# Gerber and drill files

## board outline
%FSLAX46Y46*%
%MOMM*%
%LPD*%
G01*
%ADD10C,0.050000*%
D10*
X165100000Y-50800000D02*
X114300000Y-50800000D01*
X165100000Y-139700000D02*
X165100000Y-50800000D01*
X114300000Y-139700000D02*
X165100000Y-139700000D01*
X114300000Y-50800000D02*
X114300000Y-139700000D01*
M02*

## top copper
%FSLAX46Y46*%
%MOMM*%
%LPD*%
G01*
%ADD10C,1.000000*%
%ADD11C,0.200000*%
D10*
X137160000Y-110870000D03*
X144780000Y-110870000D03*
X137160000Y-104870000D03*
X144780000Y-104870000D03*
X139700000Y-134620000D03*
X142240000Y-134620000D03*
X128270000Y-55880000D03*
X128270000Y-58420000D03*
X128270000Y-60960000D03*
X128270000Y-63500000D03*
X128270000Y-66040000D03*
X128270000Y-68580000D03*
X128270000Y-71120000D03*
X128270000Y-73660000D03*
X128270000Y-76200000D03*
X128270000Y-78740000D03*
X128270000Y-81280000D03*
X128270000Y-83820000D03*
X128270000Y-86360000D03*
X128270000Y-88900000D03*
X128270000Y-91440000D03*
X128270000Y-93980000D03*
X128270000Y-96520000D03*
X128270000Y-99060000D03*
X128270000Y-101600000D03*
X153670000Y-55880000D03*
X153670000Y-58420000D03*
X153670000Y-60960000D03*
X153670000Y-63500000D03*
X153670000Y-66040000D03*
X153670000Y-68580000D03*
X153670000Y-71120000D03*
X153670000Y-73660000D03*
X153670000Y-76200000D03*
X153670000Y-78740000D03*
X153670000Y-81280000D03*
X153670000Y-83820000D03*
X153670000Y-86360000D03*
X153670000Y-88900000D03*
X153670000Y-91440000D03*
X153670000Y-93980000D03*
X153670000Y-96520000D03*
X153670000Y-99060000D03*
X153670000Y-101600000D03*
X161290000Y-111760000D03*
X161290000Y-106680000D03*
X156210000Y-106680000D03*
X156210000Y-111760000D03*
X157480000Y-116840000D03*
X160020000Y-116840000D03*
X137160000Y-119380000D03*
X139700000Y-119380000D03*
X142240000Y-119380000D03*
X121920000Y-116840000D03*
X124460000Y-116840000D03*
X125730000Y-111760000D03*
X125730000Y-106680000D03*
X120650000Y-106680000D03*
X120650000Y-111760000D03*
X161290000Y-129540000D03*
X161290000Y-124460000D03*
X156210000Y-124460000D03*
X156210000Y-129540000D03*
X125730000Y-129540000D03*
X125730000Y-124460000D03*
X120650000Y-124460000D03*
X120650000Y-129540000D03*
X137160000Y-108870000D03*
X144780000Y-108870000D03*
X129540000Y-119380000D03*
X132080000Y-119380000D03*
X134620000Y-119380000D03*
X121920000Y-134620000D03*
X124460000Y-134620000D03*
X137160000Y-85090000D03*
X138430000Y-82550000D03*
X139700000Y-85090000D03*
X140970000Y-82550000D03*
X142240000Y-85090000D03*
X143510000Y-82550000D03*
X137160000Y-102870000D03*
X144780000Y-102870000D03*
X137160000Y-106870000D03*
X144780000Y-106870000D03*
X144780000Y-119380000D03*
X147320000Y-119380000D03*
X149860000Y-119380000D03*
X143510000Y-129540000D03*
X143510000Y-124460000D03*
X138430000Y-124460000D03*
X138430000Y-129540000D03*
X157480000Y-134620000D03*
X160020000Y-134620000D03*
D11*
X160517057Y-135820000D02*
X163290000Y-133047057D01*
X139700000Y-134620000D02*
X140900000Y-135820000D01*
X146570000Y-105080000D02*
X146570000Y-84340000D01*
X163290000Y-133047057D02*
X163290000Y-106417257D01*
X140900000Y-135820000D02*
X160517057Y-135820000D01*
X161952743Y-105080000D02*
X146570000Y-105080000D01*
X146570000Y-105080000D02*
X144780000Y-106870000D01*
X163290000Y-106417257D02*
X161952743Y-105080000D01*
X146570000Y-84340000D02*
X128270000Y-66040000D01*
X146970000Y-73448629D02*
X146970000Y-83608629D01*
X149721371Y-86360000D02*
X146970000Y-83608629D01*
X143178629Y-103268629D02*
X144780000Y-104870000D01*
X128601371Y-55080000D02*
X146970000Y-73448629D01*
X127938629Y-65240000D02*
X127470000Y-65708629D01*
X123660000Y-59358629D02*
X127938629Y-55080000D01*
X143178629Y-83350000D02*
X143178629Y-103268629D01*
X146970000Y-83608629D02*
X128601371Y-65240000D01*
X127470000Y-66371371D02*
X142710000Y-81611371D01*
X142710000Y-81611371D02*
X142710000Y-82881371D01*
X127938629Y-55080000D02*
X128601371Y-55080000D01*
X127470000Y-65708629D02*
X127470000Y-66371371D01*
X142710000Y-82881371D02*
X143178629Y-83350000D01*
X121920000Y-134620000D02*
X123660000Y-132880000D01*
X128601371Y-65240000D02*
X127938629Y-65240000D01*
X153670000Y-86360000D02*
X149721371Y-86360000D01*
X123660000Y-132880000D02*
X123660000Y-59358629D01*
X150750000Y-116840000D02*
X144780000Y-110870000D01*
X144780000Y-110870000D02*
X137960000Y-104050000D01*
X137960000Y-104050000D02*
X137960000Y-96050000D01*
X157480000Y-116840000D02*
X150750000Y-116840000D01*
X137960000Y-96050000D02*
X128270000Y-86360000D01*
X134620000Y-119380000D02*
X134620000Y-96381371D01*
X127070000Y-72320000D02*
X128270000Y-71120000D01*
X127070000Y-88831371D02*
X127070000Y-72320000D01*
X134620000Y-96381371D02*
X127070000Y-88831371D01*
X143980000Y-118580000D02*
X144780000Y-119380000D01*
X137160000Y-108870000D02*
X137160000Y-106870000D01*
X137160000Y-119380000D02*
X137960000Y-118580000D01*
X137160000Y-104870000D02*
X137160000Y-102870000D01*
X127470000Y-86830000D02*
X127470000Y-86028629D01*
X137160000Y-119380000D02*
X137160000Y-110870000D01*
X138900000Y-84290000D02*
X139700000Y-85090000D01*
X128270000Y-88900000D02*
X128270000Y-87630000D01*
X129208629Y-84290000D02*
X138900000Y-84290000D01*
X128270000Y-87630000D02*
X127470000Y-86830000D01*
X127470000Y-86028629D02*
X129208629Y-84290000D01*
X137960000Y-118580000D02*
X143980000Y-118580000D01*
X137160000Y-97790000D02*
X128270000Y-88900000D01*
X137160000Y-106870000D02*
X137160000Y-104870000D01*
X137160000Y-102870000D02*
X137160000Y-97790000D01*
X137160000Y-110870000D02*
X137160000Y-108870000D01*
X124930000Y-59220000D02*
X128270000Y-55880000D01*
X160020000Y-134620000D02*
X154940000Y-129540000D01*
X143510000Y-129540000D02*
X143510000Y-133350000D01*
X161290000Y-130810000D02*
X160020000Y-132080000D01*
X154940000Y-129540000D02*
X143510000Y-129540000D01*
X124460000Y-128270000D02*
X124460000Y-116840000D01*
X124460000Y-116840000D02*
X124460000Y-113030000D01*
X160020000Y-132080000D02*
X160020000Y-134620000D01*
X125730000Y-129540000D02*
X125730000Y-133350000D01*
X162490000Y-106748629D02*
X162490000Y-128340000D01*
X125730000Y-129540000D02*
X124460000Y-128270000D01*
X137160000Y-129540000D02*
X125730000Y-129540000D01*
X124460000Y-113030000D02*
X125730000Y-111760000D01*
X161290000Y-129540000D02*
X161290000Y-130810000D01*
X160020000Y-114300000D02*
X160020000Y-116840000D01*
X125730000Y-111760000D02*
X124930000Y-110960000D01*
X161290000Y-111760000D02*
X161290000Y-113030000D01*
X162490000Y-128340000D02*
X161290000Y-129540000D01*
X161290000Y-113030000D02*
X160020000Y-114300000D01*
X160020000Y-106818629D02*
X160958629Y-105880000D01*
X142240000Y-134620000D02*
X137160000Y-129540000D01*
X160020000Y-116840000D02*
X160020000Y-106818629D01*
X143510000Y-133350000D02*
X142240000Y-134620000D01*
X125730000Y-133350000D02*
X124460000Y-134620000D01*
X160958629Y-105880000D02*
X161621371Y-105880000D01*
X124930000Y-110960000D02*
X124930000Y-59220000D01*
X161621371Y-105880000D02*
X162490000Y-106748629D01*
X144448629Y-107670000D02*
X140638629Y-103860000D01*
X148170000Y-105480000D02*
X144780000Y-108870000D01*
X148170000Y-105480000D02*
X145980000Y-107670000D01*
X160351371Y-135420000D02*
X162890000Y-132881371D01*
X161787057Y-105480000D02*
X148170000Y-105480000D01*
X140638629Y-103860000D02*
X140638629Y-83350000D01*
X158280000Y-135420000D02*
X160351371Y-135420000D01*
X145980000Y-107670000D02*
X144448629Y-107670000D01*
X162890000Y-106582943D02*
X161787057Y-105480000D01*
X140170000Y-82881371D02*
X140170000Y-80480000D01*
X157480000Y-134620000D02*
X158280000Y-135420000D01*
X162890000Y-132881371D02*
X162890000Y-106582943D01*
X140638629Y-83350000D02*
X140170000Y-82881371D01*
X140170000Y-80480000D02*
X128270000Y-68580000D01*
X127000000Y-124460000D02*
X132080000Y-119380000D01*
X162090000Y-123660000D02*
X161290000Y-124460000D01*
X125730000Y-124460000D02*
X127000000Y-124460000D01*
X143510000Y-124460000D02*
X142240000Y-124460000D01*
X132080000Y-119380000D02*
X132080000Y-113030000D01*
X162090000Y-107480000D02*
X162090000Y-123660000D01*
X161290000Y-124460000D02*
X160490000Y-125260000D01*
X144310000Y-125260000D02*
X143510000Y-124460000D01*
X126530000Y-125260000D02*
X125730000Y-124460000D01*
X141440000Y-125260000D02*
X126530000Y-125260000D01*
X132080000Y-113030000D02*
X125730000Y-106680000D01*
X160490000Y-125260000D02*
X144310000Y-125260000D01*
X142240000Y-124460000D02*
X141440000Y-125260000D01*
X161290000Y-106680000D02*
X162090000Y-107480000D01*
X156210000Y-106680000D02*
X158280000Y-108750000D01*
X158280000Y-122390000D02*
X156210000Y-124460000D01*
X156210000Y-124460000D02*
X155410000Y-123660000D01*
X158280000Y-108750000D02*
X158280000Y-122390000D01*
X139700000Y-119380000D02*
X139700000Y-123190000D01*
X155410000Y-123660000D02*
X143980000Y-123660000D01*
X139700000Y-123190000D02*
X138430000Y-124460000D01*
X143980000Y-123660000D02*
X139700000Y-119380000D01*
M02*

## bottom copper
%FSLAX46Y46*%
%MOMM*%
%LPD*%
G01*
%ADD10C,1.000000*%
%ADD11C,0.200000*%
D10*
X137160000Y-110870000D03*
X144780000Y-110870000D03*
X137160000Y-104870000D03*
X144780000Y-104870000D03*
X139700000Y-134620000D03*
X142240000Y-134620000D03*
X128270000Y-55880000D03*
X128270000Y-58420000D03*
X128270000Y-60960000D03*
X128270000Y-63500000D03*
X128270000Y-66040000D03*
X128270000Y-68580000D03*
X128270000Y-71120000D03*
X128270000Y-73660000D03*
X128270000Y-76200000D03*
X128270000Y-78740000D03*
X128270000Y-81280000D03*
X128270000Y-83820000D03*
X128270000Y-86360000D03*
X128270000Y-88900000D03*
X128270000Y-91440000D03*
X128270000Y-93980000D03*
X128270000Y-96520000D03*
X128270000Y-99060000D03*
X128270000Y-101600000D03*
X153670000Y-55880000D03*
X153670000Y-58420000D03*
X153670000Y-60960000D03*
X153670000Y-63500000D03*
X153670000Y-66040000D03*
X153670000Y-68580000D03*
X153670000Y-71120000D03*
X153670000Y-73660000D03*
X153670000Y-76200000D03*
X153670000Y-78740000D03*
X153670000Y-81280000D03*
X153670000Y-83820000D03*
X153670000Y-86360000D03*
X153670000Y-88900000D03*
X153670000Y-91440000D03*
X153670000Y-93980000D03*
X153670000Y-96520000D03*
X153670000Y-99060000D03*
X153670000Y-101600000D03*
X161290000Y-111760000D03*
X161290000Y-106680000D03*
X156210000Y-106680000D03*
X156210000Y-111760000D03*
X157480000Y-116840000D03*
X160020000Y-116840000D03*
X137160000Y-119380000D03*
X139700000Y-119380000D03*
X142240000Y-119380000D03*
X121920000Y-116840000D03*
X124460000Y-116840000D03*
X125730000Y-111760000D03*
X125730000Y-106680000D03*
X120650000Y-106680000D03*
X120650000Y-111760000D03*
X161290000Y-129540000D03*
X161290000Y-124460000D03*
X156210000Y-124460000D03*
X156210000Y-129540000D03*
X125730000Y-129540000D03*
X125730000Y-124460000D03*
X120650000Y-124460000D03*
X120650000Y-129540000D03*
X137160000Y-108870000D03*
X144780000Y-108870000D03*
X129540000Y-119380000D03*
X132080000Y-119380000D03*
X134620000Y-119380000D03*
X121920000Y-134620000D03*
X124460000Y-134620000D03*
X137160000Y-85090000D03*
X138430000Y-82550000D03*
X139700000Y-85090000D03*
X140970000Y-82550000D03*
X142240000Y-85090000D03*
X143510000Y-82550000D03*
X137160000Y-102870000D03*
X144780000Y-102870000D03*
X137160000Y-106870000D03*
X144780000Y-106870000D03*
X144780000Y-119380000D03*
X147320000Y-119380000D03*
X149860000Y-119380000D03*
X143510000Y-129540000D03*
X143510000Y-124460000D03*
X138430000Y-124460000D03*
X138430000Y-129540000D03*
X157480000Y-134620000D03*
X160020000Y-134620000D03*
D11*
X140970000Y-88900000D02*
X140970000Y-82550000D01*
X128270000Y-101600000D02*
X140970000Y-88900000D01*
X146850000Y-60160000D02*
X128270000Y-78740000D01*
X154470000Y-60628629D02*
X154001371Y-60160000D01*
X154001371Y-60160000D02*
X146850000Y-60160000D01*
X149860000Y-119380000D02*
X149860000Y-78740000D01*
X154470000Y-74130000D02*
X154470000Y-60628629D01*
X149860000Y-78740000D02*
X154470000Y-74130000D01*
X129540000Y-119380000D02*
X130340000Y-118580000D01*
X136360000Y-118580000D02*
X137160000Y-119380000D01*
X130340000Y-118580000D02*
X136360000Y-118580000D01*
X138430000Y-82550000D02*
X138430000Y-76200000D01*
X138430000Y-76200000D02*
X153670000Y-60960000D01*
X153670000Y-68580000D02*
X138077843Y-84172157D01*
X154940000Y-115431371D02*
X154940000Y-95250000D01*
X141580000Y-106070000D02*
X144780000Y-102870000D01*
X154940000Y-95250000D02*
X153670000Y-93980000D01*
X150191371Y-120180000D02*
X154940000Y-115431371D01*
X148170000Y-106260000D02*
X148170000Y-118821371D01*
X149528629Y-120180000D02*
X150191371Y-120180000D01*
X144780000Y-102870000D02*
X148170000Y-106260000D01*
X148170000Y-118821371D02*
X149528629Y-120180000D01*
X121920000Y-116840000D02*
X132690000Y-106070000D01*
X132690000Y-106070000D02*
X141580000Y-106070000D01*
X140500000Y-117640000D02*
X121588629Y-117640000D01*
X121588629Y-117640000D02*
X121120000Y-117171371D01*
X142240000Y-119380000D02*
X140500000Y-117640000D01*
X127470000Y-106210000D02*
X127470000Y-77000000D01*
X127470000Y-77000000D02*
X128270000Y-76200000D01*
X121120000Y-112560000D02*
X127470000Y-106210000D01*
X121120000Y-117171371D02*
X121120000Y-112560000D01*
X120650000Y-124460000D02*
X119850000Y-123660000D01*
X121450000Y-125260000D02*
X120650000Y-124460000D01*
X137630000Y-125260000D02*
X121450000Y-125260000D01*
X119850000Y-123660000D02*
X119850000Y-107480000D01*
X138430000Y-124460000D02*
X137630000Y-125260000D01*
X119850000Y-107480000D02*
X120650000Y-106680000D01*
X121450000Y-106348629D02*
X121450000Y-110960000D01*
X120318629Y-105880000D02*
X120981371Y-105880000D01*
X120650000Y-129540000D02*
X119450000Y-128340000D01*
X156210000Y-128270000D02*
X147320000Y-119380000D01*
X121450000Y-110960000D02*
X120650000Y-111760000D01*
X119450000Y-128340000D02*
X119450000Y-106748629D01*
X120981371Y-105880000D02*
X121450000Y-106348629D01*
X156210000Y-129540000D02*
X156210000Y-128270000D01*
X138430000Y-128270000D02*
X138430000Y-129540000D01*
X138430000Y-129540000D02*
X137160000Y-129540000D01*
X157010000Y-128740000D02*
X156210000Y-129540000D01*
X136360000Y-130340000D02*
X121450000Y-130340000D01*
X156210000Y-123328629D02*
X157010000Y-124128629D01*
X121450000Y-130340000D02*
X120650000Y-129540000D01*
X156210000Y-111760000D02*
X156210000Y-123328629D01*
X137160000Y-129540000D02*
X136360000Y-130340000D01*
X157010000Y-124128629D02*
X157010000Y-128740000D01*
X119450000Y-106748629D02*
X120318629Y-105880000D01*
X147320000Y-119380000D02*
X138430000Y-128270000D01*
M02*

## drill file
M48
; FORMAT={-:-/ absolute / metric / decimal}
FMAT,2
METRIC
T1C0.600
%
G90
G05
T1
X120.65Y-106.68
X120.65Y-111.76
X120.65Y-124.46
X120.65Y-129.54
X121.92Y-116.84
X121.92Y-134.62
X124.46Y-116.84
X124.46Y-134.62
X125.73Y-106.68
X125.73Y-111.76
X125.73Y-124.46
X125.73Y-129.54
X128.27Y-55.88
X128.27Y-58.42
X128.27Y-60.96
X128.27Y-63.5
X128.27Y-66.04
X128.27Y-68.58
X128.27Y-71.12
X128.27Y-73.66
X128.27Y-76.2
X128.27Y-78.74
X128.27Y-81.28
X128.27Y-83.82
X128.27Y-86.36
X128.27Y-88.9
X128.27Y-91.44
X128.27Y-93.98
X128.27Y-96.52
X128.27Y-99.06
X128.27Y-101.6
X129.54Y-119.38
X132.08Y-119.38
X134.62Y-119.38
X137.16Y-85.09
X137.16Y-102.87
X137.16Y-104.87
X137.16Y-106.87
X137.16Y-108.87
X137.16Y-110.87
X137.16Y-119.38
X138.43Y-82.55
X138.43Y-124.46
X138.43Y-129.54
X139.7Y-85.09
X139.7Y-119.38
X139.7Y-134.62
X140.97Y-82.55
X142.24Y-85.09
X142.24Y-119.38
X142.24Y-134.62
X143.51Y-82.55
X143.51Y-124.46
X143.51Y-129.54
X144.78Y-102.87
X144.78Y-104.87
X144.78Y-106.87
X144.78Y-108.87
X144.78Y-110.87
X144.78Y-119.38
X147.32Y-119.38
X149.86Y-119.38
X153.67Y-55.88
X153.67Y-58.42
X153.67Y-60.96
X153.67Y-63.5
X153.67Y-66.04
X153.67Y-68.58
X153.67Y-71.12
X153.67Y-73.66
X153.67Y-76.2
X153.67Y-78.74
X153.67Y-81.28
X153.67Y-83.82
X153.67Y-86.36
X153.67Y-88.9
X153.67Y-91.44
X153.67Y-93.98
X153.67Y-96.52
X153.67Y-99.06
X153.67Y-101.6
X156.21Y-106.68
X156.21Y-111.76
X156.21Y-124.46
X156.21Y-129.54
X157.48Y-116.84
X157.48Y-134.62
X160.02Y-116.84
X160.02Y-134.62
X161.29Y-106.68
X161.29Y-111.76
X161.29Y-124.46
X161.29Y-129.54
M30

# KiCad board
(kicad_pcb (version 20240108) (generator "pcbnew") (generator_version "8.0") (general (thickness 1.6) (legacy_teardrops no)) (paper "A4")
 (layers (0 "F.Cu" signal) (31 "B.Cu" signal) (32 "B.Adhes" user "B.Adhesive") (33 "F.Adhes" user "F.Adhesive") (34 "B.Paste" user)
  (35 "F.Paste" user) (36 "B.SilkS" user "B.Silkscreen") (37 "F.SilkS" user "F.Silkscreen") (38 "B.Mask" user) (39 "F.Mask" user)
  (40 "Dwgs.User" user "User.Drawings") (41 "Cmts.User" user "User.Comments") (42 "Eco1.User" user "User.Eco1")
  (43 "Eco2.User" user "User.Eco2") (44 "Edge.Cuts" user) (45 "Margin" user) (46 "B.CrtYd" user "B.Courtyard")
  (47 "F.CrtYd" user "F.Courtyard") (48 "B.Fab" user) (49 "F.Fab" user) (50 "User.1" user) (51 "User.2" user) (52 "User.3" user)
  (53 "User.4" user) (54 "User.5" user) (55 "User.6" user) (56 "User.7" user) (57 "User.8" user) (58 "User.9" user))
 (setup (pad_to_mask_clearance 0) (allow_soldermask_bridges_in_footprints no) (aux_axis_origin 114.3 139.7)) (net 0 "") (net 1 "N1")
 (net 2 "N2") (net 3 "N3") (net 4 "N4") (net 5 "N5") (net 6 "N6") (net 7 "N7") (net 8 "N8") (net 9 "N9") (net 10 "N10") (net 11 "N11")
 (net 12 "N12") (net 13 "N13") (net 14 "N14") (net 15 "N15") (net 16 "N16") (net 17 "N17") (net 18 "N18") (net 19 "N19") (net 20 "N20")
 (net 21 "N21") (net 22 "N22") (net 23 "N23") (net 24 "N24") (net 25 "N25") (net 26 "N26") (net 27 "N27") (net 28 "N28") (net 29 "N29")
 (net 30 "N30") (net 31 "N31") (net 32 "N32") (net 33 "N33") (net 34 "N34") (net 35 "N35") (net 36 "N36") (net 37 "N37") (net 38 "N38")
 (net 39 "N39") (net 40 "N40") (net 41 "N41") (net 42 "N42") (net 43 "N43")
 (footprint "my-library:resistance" (layer "F.Cu") (at 139.7 110.87)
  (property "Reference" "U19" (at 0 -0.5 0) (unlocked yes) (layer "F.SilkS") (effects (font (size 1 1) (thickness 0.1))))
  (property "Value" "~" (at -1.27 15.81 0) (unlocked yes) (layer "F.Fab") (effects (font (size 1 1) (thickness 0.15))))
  (pad "1" thru_hole circle (at -2.54 0) (size 1 1) (drill 0.6) (layers "*.Cu" "*.Mask") (remove_unused_layers no) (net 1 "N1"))
  (pad "2" thru_hole circle (at 5.08 0) (size 1 1) (drill 0.6) (layers "*.Cu" "*.Mask") (remove_unused_layers no) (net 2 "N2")))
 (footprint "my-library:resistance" (layer "F.Cu") (at 139.7 104.87)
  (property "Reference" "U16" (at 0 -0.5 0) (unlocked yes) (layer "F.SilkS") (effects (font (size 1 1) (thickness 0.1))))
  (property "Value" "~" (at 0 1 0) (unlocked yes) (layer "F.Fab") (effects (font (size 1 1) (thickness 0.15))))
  (pad "1" thru_hole circle (at -2.54 0) (size 1 1) (drill 0.6) (layers "*.Cu" "*.Mask") (remove_unused_layers no) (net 1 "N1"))
  (pad "2" thru_hole circle (at 5.08 0) (size 1 1) (drill 0.6) (layers "*.Cu" "*.Mask") (remove_unused_layers no) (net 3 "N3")))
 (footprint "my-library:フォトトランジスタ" (layer "F.Cu") (at 139.7 134.62)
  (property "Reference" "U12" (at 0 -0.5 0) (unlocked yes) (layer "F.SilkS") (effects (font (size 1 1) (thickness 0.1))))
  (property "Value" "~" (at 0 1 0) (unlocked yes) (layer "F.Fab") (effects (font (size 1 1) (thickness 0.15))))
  (pad "1" thru_hole circle (at 0 0) (size 1 1) (drill 0.6) (layers "*.Cu" "*.Mask") (remove_unused_layers no) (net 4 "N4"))
  (pad "2" thru_hole circle (at 2.54 0) (size 1 1) (drill 0.6) (layers "*.Cu" "*.Mask") (remove_unused_layers no) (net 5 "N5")))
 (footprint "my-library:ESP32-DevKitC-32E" (layer "F.Cu") (at 140.97 76.2)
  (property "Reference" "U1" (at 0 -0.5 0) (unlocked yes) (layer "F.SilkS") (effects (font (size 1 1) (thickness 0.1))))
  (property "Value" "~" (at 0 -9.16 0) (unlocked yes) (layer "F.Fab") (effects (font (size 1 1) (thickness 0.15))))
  (pad "1" thru_hole circle (at -12.7 -20.32) (size 1 1) (drill 0.6) (layers "*.Cu" "*.Mask") (remove_unused_layers no) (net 5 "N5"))
  (pad "2" thru_hole circle (at -12.7 -17.78) (size 1 1) (drill 0.6) (layers "*.Cu" "*.Mask") (remove_unused_layers no) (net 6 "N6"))
  (pad "3" thru_hole circle (at -12.7 -15.24) (size 1 1) (drill 0.6) (layers "*.Cu" "*.Mask") (remove_unused_layers no) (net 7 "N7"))
  (pad "4" thru_hole circle (at -12.7 -12.7) (size 1 1) (drill 0.6) (layers "*.Cu" "*.Mask") (remove_unused_layers no) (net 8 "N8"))
  (pad "5" thru_hole circle (at -12.7 -10.16) (size 1 1) (drill 0.6) (layers "*.Cu" "*.Mask") (remove_unused_layers no) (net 4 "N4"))
  (pad "6" thru_hole circle (at -12.7 -7.62) (size 1 1) (drill 0.6) (layers "*.Cu" "*.Mask") (remove_unused_layers no) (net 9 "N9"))
  (pad "7" thru_hole circle (at -12.7 -5.08) (size 1 1) (drill 0.6) (layers "*.Cu" "*.Mask") (remove_unused_layers no) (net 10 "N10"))
  (pad "8" thru_hole circle (at -12.7 -2.54) (size 1 1) (drill 0.6) (layers "*.Cu" "*.Mask") (remove_unused_layers no) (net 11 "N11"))
  (pad "9" thru_hole circle (at -12.7 0) (size 1 1) (drill 0.6) (layers "*.Cu" "*.Mask") (remove_unused_layers no) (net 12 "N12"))
  (pad "10" thru_hole circle (at -12.7 2.54) (size 1 1) (drill 0.6) (layers "*.Cu" "*.Mask") (remove_unused_layers no) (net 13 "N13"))
  (pad "11" thru_hole circle (at -12.7 5.08) (size 1 1) (drill 0.6) (layers "*.Cu" "*.Mask") (remove_unused_layers no) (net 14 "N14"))
  (pad "12" thru_hole circle (at -12.7 7.62) (size 1 1) (drill 0.6) (layers "*.Cu" "*.Mask") (remove_unused_layers no) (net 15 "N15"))
  (pad "13" thru_hole circle (at -12.7 10.16) (size 1 1) (drill 0.6) (layers "*.Cu" "*.Mask") (remove_unused_layers no) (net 2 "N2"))
  (pad "14" thru_hole circle (at -12.7 12.7) (size 1 1) (drill 0.6) (layers "*.Cu" "*.Mask") (remove_unused_layers no) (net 1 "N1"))
  (pad "15" thru_hole circle (at -12.7 15.24) (size 1 1) (drill 0.6) (layers "*.Cu" "*.Mask") (remove_unused_layers no) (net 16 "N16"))
  (pad "16" thru_hole circle (at -12.7 17.78) (size 1 1) (drill 0.6) (layers "*.Cu" "*.Mask") (remove_unused_layers no) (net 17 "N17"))
  (pad "17" thru_hole circle (at -12.7 20.32) (size 1 1) (drill 0.6) (layers "*.Cu" "*.Mask") (remove_unused_layers no) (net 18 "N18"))
  (pad "18" thru_hole circle (at -12.7 22.86) (size 1 1) (drill 0.6) (layers "*.Cu" "*.Mask") (remove_unused_layers no) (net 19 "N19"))
  (pad "19" thru_hole circle (at -12.7 25.4) (size 1 1) (drill 0.6) (layers "*.Cu" "*.Mask") (remove_unused_layers no) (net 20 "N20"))
  (pad "20" thru_hole circle (at 12.7 -20.32) (size 1 1) (drill 0.6) (layers "*.Cu" "*.Mask") (remove_unused_layers no) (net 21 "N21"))
  (pad "21" thru_hole circle (at 12.7 -17.78) (size 1 1) (drill 0.6) (layers "*.Cu" "*.Mask") (remove_unused_layers no) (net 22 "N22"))
  (pad "22" thru_hole circle (at 12.7 -15.24) (size 1 1) (drill 0.6) (layers "*.Cu" "*.Mask") (remove_unused_layers no) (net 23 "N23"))
  (pad "23" thru_hole circle (at 12.7 -12.7) (size 1 1) (drill 0.6) (layers "*.Cu" "*.Mask") (remove_unused_layers no) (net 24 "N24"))
  (pad "24" thru_hole circle (at 12.7 -10.16) (size 1 1) (drill 0.6) (layers "*.Cu" "*.Mask") (remove_unused_layers no) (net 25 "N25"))
  (pad "25" thru_hole circle (at 12.7 -7.62) (size 1 1) (drill 0.6) (layers "*.Cu" "*.Mask") (remove_unused_layers no) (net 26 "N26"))
  (pad "26" thru_hole circle (at 12.7 -5.08) (size 1 1) (drill 0.6) (layers "*.Cu" "*.Mask") (remove_unused_layers no) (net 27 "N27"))
  (pad "27" thru_hole circle (at 12.7 -2.54) (size 1 1) (drill 0.6) (layers "*.Cu" "*.Mask") (remove_unused_layers no) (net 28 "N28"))
  (pad "28" thru_hole circle (at 12.7 0) (size 1 1) (drill 0.6) (layers "*.Cu" "*.Mask") (remove_unused_layers no) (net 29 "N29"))
  (pad "29" thru_hole circle (at 12.7 2.54) (size 1 1) (drill 0.6) (layers "*.Cu" "*.Mask") (remove_unused_layers no) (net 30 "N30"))
  (pad "30" thru_hole circle (at 12.7 5.08) (size 1 1) (drill 0.6) (layers "*.Cu" "*.Mask") (remove_unused_layers no) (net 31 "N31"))
  (pad "31" thru_hole circle (at 12.7 7.62) (size 1 1) (drill 0.6) (layers "*.Cu" "*.Mask") (remove_unused_layers no) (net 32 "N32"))
  (pad "32" thru_hole circle (at 12.7 10.16) (size 1 1) (drill 0.6) (layers "*.Cu" "*.Mask") (remove_unused_layers no) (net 3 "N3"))
  (pad "33" thru_hole circle (at 12.7 12.7) (size 1 1) (drill 0.6) (layers "*.Cu" "*.Mask") (remove_unused_layers no) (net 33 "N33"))
  (pad "34" thru_hole circle (at 12.7 15.24) (size 1 1) (drill 0.6) (layers "*.Cu" "*.Mask") (remove_unused_layers no) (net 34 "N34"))
  (pad "35" thru_hole circle (at 12.7 17.78) (size 1 1) (drill 0.6) (layers "*.Cu" "*.Mask") (remove_unused_layers no) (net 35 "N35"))
  (pad "36" thru_hole circle (at 12.7 20.32) (size 1 1) (drill 0.6) (layers "*.Cu" "*.Mask") (remove_unused_layers no) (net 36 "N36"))
  (pad "37" thru_hole circle (at 12.7 22.86) (size 1 1) (drill 0.6) (layers "*.Cu" "*.Mask") (remove_unused_layers no) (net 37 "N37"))
  (pad "38" thru_hole circle (at 12.7 25.4) (size 1 1) (drill 0.6) (layers "*.Cu" "*.Mask") (remove_unused_layers no) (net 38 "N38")))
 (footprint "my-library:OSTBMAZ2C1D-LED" (layer "F.Cu") (at 158.75 109.22)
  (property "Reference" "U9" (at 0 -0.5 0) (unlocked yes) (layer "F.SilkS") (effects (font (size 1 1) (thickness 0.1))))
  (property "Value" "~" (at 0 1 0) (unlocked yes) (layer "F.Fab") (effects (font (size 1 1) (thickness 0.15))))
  (pad "1" thru_hole circle (at 2.54 2.54) (size 1 1) (drill 0.6) (layers "*.Cu" "*.Mask") (remove_unused_layers no) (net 5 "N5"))
  (pad "2" thru_hole circle (at 2.54 -2.54) (size 1 1) (drill 0.6) (layers "*.Cu" "*.Mask") (remove_unused_layers no) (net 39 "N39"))
  (pad "3" thru_hole circle (at -2.54 -2.54) (size 1 1) (drill 0.6) (layers "*.Cu" "*.Mask") (remove_unused_layers no) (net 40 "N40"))
  (pad "4" thru_hole circle (at -2.54 2.54) (size 1 1) (drill 0.6) (layers "*.Cu" "*.Mask") (remove_unused_layers no) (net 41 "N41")))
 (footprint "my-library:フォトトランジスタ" (layer "F.Cu") (at 157.48 116.84)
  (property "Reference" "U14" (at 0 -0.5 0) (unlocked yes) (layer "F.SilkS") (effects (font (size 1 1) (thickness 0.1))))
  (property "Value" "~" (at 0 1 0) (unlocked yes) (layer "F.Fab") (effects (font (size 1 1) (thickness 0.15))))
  (pad "1" thru_hole circle (at 0 0) (size 1 1) (drill 0.6) (layers "*.Cu" "*.Mask") (remove_unused_layers no) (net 2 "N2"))
  (pad "2" thru_hole circle (at 2.54 0) (size 1 1) (drill 0.6) (layers "*.Cu" "*.Mask") (remove_unused_layers no) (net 5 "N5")))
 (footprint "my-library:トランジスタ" (layer "F.Cu") (at 139.7 116.84)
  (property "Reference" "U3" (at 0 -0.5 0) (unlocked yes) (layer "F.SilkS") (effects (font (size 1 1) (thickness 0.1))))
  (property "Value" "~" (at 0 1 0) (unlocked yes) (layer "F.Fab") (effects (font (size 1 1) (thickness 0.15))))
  (pad "1" thru_hole circle (at -2.54 2.54) (size 1 1) (drill 0.6) (layers "*.Cu" "*.Mask") (remove_unused_layers no) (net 1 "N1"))
  (pad "2" thru_hole circle (at 0 2.54) (size 1 1) (drill 0.6) (layers "*.Cu" "*.Mask") (remove_unused_layers no) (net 40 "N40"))
  (pad "3" thru_hole circle (at 2.54 2.54) (size 1 1) (drill 0.6) (layers "*.Cu" "*.Mask") (remove_unused_layers no) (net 12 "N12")))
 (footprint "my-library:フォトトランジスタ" (layer "F.Cu") (at 121.92 116.84)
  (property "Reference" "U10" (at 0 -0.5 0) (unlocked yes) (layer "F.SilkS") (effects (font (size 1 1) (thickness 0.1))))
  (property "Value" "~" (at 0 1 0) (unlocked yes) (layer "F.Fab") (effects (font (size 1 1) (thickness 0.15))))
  (pad "1" thru_hole circle (at 0 0) (size 1 1) (drill 0.6) (layers "*.Cu" "*.Mask") (remove_unused_layers no) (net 35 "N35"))
  (pad "2" thru_hole circle (at 2.54 0) (size 1 1) (drill 0.6) (layers "*.Cu" "*.Mask") (remove_unused_layers no) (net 5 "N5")))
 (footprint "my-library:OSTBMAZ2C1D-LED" (layer "F.Cu") (at 123.19 109.22)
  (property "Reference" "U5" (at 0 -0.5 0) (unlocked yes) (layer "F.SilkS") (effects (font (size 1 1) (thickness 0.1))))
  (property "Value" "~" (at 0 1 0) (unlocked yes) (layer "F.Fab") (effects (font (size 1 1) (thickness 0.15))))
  (pad "1" thru_hole circle (at 2.54 2.54) (size 1 1) (drill 0.6) (layers "*.Cu" "*.Mask") (remove_unused_layers no) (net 5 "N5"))
  (pad "2" thru_hole circle (at 2.54 -2.54) (size 1 1) (drill 0.6) (layers "*.Cu" "*.Mask") (remove_unused_layers no) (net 39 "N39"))
  (pad "3" thru_hole circle (at -2.54 -2.54) (size 1 1) (drill 0.6) (layers "*.Cu" "*.Mask") (remove_unused_layers no) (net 40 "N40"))
  (pad "4" thru_hole circle (at -2.54 2.54) (size 1 1) (drill 0.6) (layers "*.Cu" "*.Mask") (remove_unused_layers no) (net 41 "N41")))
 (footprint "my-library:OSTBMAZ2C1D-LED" (layer "F.Cu") (at 158.75 127)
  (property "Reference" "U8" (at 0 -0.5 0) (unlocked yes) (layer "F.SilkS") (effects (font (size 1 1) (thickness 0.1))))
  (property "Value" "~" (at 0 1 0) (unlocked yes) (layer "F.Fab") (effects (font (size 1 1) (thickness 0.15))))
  (pad "1" thru_hole circle (at 2.54 2.54) (size 1 1) (drill 0.6) (layers "*.Cu" "*.Mask") (remove_unused_layers no) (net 5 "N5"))
  (pad "2" thru_hole circle (at 2.54 -2.54) (size 1 1) (drill 0.6) (layers "*.Cu" "*.Mask") (remove_unused_layers no) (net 39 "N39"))
  (pad "3" thru_hole circle (at -2.54 -2.54) (size 1 1) (drill 0.6) (layers "*.Cu" "*.Mask") (remove_unused_layers no) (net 40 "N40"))
  (pad "4" thru_hole circle (at -2.54 2.54) (size 1 1) (drill 0.6) (layers "*.Cu" "*.Mask") (remove_unused_layers no) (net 41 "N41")))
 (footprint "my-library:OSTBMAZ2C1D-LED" (layer "F.Cu") (at 123.19 127)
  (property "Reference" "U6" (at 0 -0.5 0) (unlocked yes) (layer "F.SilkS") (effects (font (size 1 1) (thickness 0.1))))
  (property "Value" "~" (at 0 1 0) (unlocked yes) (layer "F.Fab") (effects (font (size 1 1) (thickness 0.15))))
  (pad "1" thru_hole circle (at 2.54 2.54) (size 1 1) (drill 0.6) (layers "*.Cu" "*.Mask") (remove_unused_layers no) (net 5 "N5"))
  (pad "2" thru_hole circle (at 2.54 -2.54) (size 1 1) (drill 0.6) (layers "*.Cu" "*.Mask") (remove_unused_layers no) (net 39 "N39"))
  (pad "3" thru_hole circle (at -2.54 -2.54) (size 1 1) (drill 0.6) (layers "*.Cu" "*.Mask") (remove_unused_layers no) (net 40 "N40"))
  (pad "4" thru_hole circle (at -2.54 2.54) (size 1 1) (drill 0.6) (layers "*.Cu" "*.Mask") (remove_unused_layers no) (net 41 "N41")))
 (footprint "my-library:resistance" (layer "F.Cu") (at 139.7 108.87)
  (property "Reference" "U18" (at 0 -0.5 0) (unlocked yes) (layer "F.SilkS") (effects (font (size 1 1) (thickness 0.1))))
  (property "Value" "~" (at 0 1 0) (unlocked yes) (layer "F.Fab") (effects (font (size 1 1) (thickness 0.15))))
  (pad "1" thru_hole circle (at -2.54 0) (size 1 1) (drill 0.6) (layers "*.Cu" "*.Mask") (remove_unused_layers no) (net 1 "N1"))
  (pad "2" thru_hole circle (at 5.08 0) (size 1 1) (drill 0.6) (layers "*.Cu" "*.Mask") (remove_unused_layers no) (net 9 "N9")))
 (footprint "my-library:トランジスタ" (layer "F.Cu") (at 132.08 116.84)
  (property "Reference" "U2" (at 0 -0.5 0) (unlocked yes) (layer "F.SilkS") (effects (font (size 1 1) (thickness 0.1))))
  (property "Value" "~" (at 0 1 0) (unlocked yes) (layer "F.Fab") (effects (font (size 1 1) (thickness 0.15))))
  (pad "1" thru_hole circle (at -2.54 2.54) (size 1 1) (drill 0.6) (layers "*.Cu" "*.Mask") (remove_unused_layers no) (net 1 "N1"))
  (pad "2" thru_hole circle (at 0 2.54) (size 1 1) (drill 0.6) (layers "*.Cu" "*.Mask") (remove_unused_layers no) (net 39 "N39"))
  (pad "3" thru_hole circle (at 2.54 2.54) (size 1 1) (drill 0.6) (layers "*.Cu" "*.Mask") (remove_unused_layers no) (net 10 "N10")))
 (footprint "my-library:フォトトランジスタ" (layer "F.Cu") (at 121.92 134.62)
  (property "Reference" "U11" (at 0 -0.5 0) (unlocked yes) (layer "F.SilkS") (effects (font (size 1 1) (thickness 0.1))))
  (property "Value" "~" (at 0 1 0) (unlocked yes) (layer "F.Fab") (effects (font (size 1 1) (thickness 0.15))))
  (pad "1" thru_hole circle (at 0 0) (size 1 1) (drill 0.6) (layers "*.Cu" "*.Mask") (remove_unused_layers no) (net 3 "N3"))
  (pad "2" thru_hole circle (at 2.54 0) (size 1 1) (drill 0.6) (layers "*.Cu" "*.Mask") (remove_unused_layers no) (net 5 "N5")))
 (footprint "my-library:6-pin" (layer "F.Cu") (at 139.7 82.55)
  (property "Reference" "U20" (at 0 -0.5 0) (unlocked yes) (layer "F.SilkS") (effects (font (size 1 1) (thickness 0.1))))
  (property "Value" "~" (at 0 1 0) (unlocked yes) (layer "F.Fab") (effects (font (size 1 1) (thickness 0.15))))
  (pad "1" thru_hole circle (at -2.54 2.54) (size 1 1) (drill 0.6) (layers "*.Cu" "*.Mask") (remove_unused_layers no) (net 26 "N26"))
  (pad "2" thru_hole circle (at -1.27 0) (size 1 1) (drill 0.6) (layers "*.Cu" "*.Mask") (remove_unused_layers no) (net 23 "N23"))
  (pad "3" thru_hole circle (at 0 2.54) (size 1 1) (drill 0.6) (layers "*.Cu" "*.Mask") (remove_unused_layers no) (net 1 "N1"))
  (pad "4" thru_hole circle (at 1.27 0) (size 1 1) (drill 0.6) (layers "*.Cu" "*.Mask") (remove_unused_layers no) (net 20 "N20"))
  (pad "5" thru_hole circle (at 2.54 2.54) (size 1 1) (drill 0.6) (layers "*.Cu" "*.Mask") (remove_unused_layers no) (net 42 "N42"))
  (pad "6" thru_hole circle (at 3.81 0) (size 1 1) (drill 0.6) (layers "*.Cu" "*.Mask") (remove_unused_layers no) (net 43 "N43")))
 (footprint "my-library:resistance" (layer "F.Cu") (at 139.7 102.87)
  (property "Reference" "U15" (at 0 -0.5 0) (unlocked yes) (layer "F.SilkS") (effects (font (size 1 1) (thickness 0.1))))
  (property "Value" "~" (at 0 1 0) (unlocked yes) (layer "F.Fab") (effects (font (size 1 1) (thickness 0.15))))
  (pad "1" thru_hole circle (at -2.54 0) (size 1 1) (drill 0.6) (layers "*.Cu" "*.Mask") (remove_unused_layers no) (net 1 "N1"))
  (pad "2" thru_hole circle (at 5.08 0) (size 1 1) (drill 0.6) (layers "*.Cu" "*.Mask") (remove_unused_layers no) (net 35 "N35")))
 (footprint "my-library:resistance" (layer "F.Cu") (at 139.7 106.87)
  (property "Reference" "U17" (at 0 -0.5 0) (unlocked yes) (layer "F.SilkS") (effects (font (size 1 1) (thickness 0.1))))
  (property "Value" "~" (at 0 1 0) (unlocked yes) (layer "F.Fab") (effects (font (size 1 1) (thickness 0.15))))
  (pad "1" thru_hole circle (at -2.54 0) (size 1 1) (drill 0.6) (layers "*.Cu" "*.Mask") (remove_unused_layers no) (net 1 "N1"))
  (pad "2" thru_hole circle (at 5.08 0) (size 1 1) (drill 0.6) (layers "*.Cu" "*.Mask") (remove_unused_layers no) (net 4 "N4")))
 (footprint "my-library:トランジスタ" (layer "F.Cu") (at 147.32 116.84)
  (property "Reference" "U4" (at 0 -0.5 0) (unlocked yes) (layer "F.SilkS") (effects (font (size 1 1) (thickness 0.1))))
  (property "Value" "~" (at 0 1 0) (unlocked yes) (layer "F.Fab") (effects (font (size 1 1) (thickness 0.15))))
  (pad "1" thru_hole circle (at -2.54 2.54) (size 1 1) (drill 0.6) (layers "*.Cu" "*.Mask") (remove_unused_layers no) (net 1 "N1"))
  (pad "2" thru_hole circle (at 0 2.54) (size 1 1) (drill 0.6) (layers "*.Cu" "*.Mask") (remove_unused_layers no) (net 41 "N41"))
  (pad "3" thru_hole circle (at 2.54 2.54) (size 1 1) (drill 0.6) (layers "*.Cu" "*.Mask") (remove_unused_layers no) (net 13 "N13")))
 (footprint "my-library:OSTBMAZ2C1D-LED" (layer "F.Cu") (at 140.97 127)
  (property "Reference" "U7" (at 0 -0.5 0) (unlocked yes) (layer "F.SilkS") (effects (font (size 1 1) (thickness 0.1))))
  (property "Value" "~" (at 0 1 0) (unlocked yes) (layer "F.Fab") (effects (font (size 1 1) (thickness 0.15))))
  (pad "1" thru_hole circle (at 2.54 2.54) (size 1 1) (drill 0.6) (layers "*.Cu" "*.Mask") (remove_unused_layers no) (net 5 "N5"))
  (pad "2" thru_hole circle (at 2.54 -2.54) (size 1 1) (drill 0.6) (layers "*.Cu" "*.Mask") (remove_unused_layers no) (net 39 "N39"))
  (pad "3" thru_hole circle (at -2.54 -2.54) (size 1 1) (drill 0.6) (layers "*.Cu" "*.Mask") (remove_unused_layers no) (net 40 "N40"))
  (pad "4" thru_hole circle (at -2.54 2.54) (size 1 1) (drill 0.6) (layers "*.Cu" "*.Mask") (remove_unused_layers no) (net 41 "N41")))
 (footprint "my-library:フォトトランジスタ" (layer "F.Cu") (at 157.48 134.62)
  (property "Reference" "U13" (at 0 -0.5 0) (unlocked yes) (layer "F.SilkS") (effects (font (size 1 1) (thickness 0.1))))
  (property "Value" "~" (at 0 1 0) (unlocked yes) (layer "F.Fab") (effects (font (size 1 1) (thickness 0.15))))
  (pad "1" thru_hole circle (at 0 0) (size 1 1) (drill 0.6) (layers "*.Cu" "*.Mask") (remove_unused_layers no) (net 9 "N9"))
  (pad "2" thru_hole circle (at 2.54 0) (size 1 1) (drill 0.6) (layers "*.Cu" "*.Mask") (remove_unused_layers no) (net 5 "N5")))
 (gr_line (start 165.1 50.8) (end 114.3 50.8) (stroke (width 0.05) (type default)) (layer "Edge.Cuts"))
 (gr_line (start 165.1 139.7) (end 165.1 50.8) (stroke (width 0.05) (type default)) (layer "Edge.Cuts"))
 (gr_line (start 114.3 139.7) (end 165.1 139.7) (stroke (width 0.05) (type default)) (layer "Edge.Cuts"))
 (gr_line (start 114.3 50.8) (end 114.3 139.7) (stroke (width 0.05) (type default)) (layer "Edge.Cuts"))
 (segment (start 140.97 88.9) (end 140.97 82.55) (width 0.2) (layer "B.Cu") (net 20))
 (segment (start 128.27 101.6) (end 140.97 88.9) (width 0.2) (layer "B.Cu") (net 20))
 (segment (start 160.517057 135.82) (end 163.29 133.047057) (width 0.2) (layer "F.Cu") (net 4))
 (segment (start 139.7 134.62) (end 140.9 135.82) (width 0.2) (layer "F.Cu") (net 4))
 (segment (start 146.57 105.08) (end 146.57 84.34) (width 0.2) (layer "F.Cu") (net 4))
 (segment (start 163.29 133.047057) (end 163.29 106.417257) (width 0.2) (layer "F.Cu") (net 4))
 (segment (start 140.9 135.82) (end 160.517057 135.82) (width 0.2) (layer "F.Cu") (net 4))
 (segment (start 161.952743 105.08) (end 146.57 105.08) (width 0.2) (layer "F.Cu") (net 4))
 (segment (start 146.57 105.08) (end 144.78 106.87) (width 0.2) (layer "F.Cu") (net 4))
 (segment (start 163.29 106.417257) (end 161.952743 105.08) (width 0.2) (layer "F.Cu") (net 4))
 (segment (start 146.57 84.34) (end 128.27 66.04) (width 0.2) (layer "F.Cu") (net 4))
 (segment (start 146.97 73.448629) (end 146.97 83.608629) (width 0.2) (layer "F.Cu") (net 3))
 (segment (start 149.721371 86.36) (end 146.97 83.608629) (width 0.2) (layer "F.Cu") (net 3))
 (segment (start 143.178629 103.268629) (end 144.78 104.87) (width 0.2) (layer "F.Cu") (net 3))
 (segment (start 128.601371 55.08) (end 146.97 73.448629) (width 0.2) (layer "F.Cu") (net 3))
 (segment (start 127.938629 65.24) (end 127.47 65.708629) (width 0.2) (layer "F.Cu") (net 3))
 (segment (start 123.66 59.358629) (end 127.938629 55.08) (width 0.2) (layer "F.Cu") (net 3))
 (segment (start 143.178629 83.35) (end 143.178629 103.268629) (width 0.2) (layer "F.Cu") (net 3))
 (segment (start 146.97 83.608629) (end 128.601371 65.24) (width 0.2) (layer "F.Cu") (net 3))
 (segment (start 127.47 66.371371) (end 142.71 81.611371) (width 0.2) (layer "F.Cu") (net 3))
 (segment (start 142.71 81.611371) (end 142.71 82.881371) (width 0.2) (layer "F.Cu") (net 3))
 (segment (start 127.938629 55.08) (end 128.601371 55.08) (width 0.2) (layer "F.Cu") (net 3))
 (segment (start 127.47 65.708629) (end 127.47 66.371371) (width 0.2) (layer "F.Cu") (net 3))
 (segment (start 142.71 82.881371) (end 143.178629 83.35) (width 0.2) (layer "F.Cu") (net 3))
 (segment (start 121.92 134.62) (end 123.66 132.88) (width 0.2) (layer "F.Cu") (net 3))
 (segment (start 128.601371 65.24) (end 127.938629 65.24) (width 0.2) (layer "F.Cu") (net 3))
 (segment (start 153.67 86.36) (end 149.721371 86.36) (width 0.2) (layer "F.Cu") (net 3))
 (segment (start 123.66 132.88) (end 123.66 59.358629) (width 0.2) (layer "F.Cu") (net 3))
 (segment (start 150.75 116.84) (end 144.78 110.87) (width 0.2) (layer "F.Cu") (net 2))
 (segment (start 144.78 110.87) (end 137.96 104.05) (width 0.2) (layer "F.Cu") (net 2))
 (segment (start 137.96 104.05) (end 137.96 96.05) (width 0.2) (layer "F.Cu") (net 2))
 (segment (start 157.48 116.84) (end 150.75 116.84) (width 0.2) (layer "F.Cu") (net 2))
 (segment (start 137.96 96.05) (end 128.27 86.36) (width 0.2) (layer "F.Cu") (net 2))
 (segment (start 146.85 60.16) (end 128.27 78.74) (width 0.2) (layer "B.Cu") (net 13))
 (segment (start 154.47 60.628629) (end 154.001371 60.16) (width 0.2) (layer "B.Cu") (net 13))
 (segment (start 154.001371 60.16) (end 146.85 60.16) (width 0.2) (layer "B.Cu") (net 13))
 (segment (start 149.86 119.38) (end 149.86 78.74) (width 0.2) (layer "B.Cu") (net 13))
 (segment (start 154.47 74.13) (end 154.47 60.628629) (width 0.2) (layer "B.Cu") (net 13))
 (segment (start 149.86 78.74) (end 154.47 74.13) (width 0.2) (layer "B.Cu") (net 13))
 (segment (start 134.62 119.38) (end 134.62 96.381371) (width 0.2) (layer "F.Cu") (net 10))
 (segment (start 127.07 72.32) (end 128.27 71.12) (width 0.2) (layer "F.Cu") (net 10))
 (segment (start 127.07 88.831371) (end 127.07 72.32) (width 0.2) (layer "F.Cu") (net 10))
 (segment (start 134.62 96.381371) (end 127.07 88.831371) (width 0.2) (layer "F.Cu") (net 10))
 (segment (start 143.98 118.58) (end 144.78 119.38) (width 0.2) (layer "F.Cu") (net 1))
 (segment (start 137.16 108.87) (end 137.16 106.87) (width 0.2) (layer "F.Cu") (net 1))
 (segment (start 137.16 119.38) (end 137.96 118.58) (width 0.2) (layer "F.Cu") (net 1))
 (segment (start 137.16 104.87) (end 137.16 102.87) (width 0.2) (layer "F.Cu") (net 1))
 (segment (start 127.47 86.83) (end 127.47 86.028629) (width 0.2) (layer "F.Cu") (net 1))
 (segment (start 137.16 119.38) (end 137.16 110.87) (width 0.2) (layer "F.Cu") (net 1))
 (segment (start 138.9 84.29) (end 139.7 85.09) (width 0.2) (layer "F.Cu") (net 1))
 (segment (start 128.27 88.9) (end 128.27 87.63) (width 0.2) (layer "F.Cu") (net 1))
 (segment (start 129.208629 84.29) (end 138.9 84.29) (width 0.2) (layer "F.Cu") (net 1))
 (segment (start 128.27 87.63) (end 127.47 86.83) (width 0.2) (layer "F.Cu") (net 1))
 (segment (start 127.47 86.028629) (end 129.208629 84.29) (width 0.2) (layer "F.Cu") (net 1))
 (segment (start 137.96 118.58) (end 143.98 118.58) (width 0.2) (layer "F.Cu") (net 1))
 (segment (start 137.16 97.79) (end 128.27 88.9) (width 0.2) (layer "F.Cu") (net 1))
 (segment (start 137.16 106.87) (end 137.16 104.87) (width 0.2) (layer "F.Cu") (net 1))
 (segment (start 137.16 102.87) (end 137.16 97.79) (width 0.2) (layer "F.Cu") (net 1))
 (segment (start 137.16 110.87) (end 137.16 108.87) (width 0.2) (layer "F.Cu") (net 1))
 (segment (start 129.54 119.38) (end 130.34 118.58) (width 0.2) (layer "B.Cu") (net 1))
 (segment (start 136.36 118.58) (end 137.16 119.38) (width 0.2) (layer "B.Cu") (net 1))
 (segment (start 130.34 118.58) (end 136.36 118.58) (width 0.2) (layer "B.Cu") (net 1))
 (segment (start 124.93 59.22) (end 128.27 55.88) (width 0.2) (layer "F.Cu") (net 5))
 (segment (start 160.02 134.62) (end 154.94 129.54) (width 0.2) (layer "F.Cu") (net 5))
 (segment (start 143.51 129.54) (end 143.51 133.35) (width 0.2) (layer "F.Cu") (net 5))
 (segment (start 161.29 130.81) (end 160.02 132.08) (width 0.2) (layer "F.Cu") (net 5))
 (segment (start 154.94 129.54) (end 143.51 129.54) (width 0.2) (layer "F.Cu") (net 5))
 (segment (start 124.46 128.27) (end 124.46 116.84) (width 0.2) (layer "F.Cu") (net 5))
 (segment (start 124.46 116.84) (end 124.46 113.03) (width 0.2) (layer "F.Cu") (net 5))
 (segment (start 160.02 132.08) (end 160.02 134.62) (width 0.2) (layer "F.Cu") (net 5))
 (segment (start 125.73 129.54) (end 125.73 133.35) (width 0.2) (layer "F.Cu") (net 5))
 (segment (start 162.49 106.748629) (end 162.49 128.34) (width 0.2) (layer "F.Cu") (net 5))
 (segment (start 125.73 129.54) (end 124.46 128.27) (width 0.2) (layer "F.Cu") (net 5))
 (segment (start 137.16 129.54) (end 125.73 129.54) (width 0.2) (layer "F.Cu") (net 5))
 (segment (start 124.46 113.03) (end 125.73 111.76) (width 0.2) (layer "F.Cu") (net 5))
 (segment (start 161.29 129.54) (end 161.29 130.81) (width 0.2) (layer "F.Cu") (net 5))
 (segment (start 160.02 114.3) (end 160.02 116.84) (width 0.2) (layer "F.Cu") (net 5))
 (segment (start 125.73 111.76) (end 124.93 110.96) (width 0.2) (layer "F.Cu") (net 5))
 (segment (start 161.29 111.76) (end 161.29 113.03) (width 0.2) (layer "F.Cu") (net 5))
 (segment (start 162.49 128.34) (end 161.29 129.54) (width 0.2) (layer "F.Cu") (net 5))
 (segment (start 161.29 113.03) (end 160.02 114.3) (width 0.2) (layer "F.Cu") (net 5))
 (segment (start 160.02 106.818629) (end 160.958629 105.88) (width 0.2) (layer "F.Cu") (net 5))
 (segment (start 142.24 134.62) (end 137.16 129.54) (width 0.2) (layer "F.Cu") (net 5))
 (segment (start 160.02 116.84) (end 160.02 106.818629) (width 0.2) (layer "F.Cu") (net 5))
 (segment (start 143.51 133.35) (end 142.24 134.62) (width 0.2) (layer "F.Cu") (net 5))
 (segment (start 125.73 133.35) (end 124.46 134.62) (width 0.2) (layer "F.Cu") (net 5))
 (segment (start 160.958629 105.88) (end 161.621371 105.88) (width 0.2) (layer "F.Cu") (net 5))
 (segment (start 124.93 110.96) (end 124.93 59.22) (width 0.2) (layer "F.Cu") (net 5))
 (segment (start 161.621371 105.88) (end 162.49 106.748629) (width 0.2) (layer "F.Cu") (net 5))
 (segment (start 138.43 82.55) (end 138.43 76.2) (width 0.2) (layer "B.Cu") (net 23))
 (segment (start 138.43 76.2) (end 153.67 60.96) (width 0.2) (layer "B.Cu") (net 23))
 (segment (start 153.67 68.58) (end 138.077843 84.172157) (width 0.2) (layer "B.Cu") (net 26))
 (segment (start 154.94 115.431371) (end 154.94 95.25) (width 0.2) (layer "B.Cu") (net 35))
 (segment (start 141.58 106.07) (end 144.78 102.87) (width 0.2) (layer "B.Cu") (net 35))
 (segment (start 154.94 95.25) (end 153.67 93.98) (width 0.2) (layer "B.Cu") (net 35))
 (segment (start 150.191371 120.18) (end 154.94 115.431371) (width 0.2) (layer "B.Cu") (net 35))
 (segment (start 148.17 106.26) (end 148.17 118.821371) (width 0.2) (layer "B.Cu") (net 35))
 (segment (start 149.528629 120.18) (end 150.191371 120.18) (width 0.2) (layer "B.Cu") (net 35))
 (segment (start 144.78 102.87) (end 148.17 106.26) (width 0.2) (layer "B.Cu") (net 35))
 (segment (start 148.17 118.821371) (end 149.528629 120.18) (width 0.2) (layer "B.Cu") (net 35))
 (segment (start 121.92 116.84) (end 132.69 106.07) (width 0.2) (layer "B.Cu") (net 35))
 (segment (start 132.69 106.07) (end 141.58 106.07) (width 0.2) (layer "B.Cu") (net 35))
 (segment (start 140.5 117.64) (end 121.588629 117.64) (width 0.2) (layer "B.Cu") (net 12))
 (segment (start 121.588629 117.64) (end 121.12 117.171371) (width 0.2) (layer "B.Cu") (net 12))
 (segment (start 142.24 119.38) (end 140.5 117.64) (width 0.2) (layer "B.Cu") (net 12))
 (segment (start 127.47 106.21) (end 127.47 77) (width 0.2) (layer "B.Cu") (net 12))
 (segment (start 127.47 77) (end 128.27 76.2) (width 0.2) (layer "B.Cu") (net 12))
 (segment (start 121.12 112.56) (end 127.47 106.21) (width 0.2) (layer "B.Cu") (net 12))
 (segment (start 121.12 117.171371) (end 121.12 112.56) (width 0.2) (layer "B.Cu") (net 12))
 (segment (start 144.448629 107.67) (end 140.638629 103.86) (width 0.2) (layer "F.Cu") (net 9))
 (segment (start 148.17 105.48) (end 144.78 108.87) (width 0.2) (layer "F.Cu") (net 9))
 (segment (start 148.17 105.48) (end 145.98 107.67) (width 0.2) (layer "F.Cu") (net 9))
 (segment (start 160.351371 135.42) (end 162.89 132.881371) (width 0.2) (layer "F.Cu") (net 9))
 (segment (start 161.787057 105.48) (end 148.17 105.48) (width 0.2) (layer "F.Cu") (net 9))
 (segment (start 140.638629 103.86) (end 140.638629 83.35) (width 0.2) (layer "F.Cu") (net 9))
 (segment (start 158.28 135.42) (end 160.351371 135.42) (width 0.2) (layer "F.Cu") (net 9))
 (segment (start 145.98 107.67) (end 144.448629 107.67) (width 0.2) (layer "F.Cu") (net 9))
 (segment (start 162.89 106.582943) (end 161.787057 105.48) (width 0.2) (layer "F.Cu") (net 9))
 (segment (start 140.17 82.881371) (end 140.17 80.48) (width 0.2) (layer "F.Cu") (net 9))
 (segment (start 157.48 134.62) (end 158.28 135.42) (width 0.2) (layer "F.Cu") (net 9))
 (segment (start 162.89 132.881371) (end 162.89 106.582943) (width 0.2) (layer "F.Cu") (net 9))
 (segment (start 140.638629 83.35) (end 140.17 82.881371) (width 0.2) (layer "F.Cu") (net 9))
 (segment (start 140.17 80.48) (end 128.27 68.58) (width 0.2) (layer "F.Cu") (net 9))
 (segment (start 127 124.46) (end 132.08 119.38) (width 0.2) (layer "F.Cu") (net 39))
 (segment (start 162.09 123.66) (end 161.29 124.46) (width 0.2) (layer "F.Cu") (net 39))
 (segment (start 125.73 124.46) (end 127 124.46) (width 0.2) (layer "F.Cu") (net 39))
 (segment (start 143.51 124.46) (end 142.24 124.46) (width 0.2) (layer "F.Cu") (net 39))
 (segment (start 132.08 119.38) (end 132.08 113.03) (width 0.2) (layer "F.Cu") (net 39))
 (segment (start 162.09 107.48) (end 162.09 123.66) (width 0.2) (layer "F.Cu") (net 39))
 (segment (start 161.29 124.46) (end 160.49 125.26) (width 0.2) (layer "F.Cu") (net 39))
 (segment (start 144.31 125.26) (end 143.51 124.46) (width 0.2) (layer "F.Cu") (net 39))
 (segment (start 126.53 125.26) (end 125.73 124.46) (width 0.2) (layer "F.Cu") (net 39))
 (segment (start 141.44 125.26) (end 126.53 125.26) (width 0.2) (layer "F.Cu") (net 39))
 (segment (start 132.08 113.03) (end 125.73 106.68) (width 0.2) (layer "F.Cu") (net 39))
 (segment (start 160.49 125.26) (end 144.31 125.26) (width 0.2) (layer "F.Cu") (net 39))
 (segment (start 142.24 124.46) (end 141.44 125.26) (width 0.2) (layer "F.Cu") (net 39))
 (segment (start 161.29 106.68) (end 162.09 107.48) (width 0.2) (layer "F.Cu") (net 39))
 (segment (start 156.21 106.68) (end 158.28 108.75) (width 0.2) (layer "F.Cu") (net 40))
 (segment (start 158.28 122.39) (end 156.21 124.46) (width 0.2) (layer "F.Cu") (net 40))
 (segment (start 156.21 124.46) (end 155.41 123.66) (width 0.2) (layer "F.Cu") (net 40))
 (segment (start 158.28 108.75) (end 158.28 122.39) (width 0.2) (layer "F.Cu") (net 40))
 (segment (start 139.7 119.38) (end 139.7 123.19) (width 0.2) (layer "F.Cu") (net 40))
 (segment (start 155.41 123.66) (end 143.98 123.66) (width 0.2) (layer "F.Cu") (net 40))
 (segment (start 139.7 123.19) (end 138.43 124.46) (width 0.2) (layer "F.Cu") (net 40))
 (segment (start 143.98 123.66) (end 139.7 119.38) (width 0.2) (layer "F.Cu") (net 40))
 (segment (start 120.65 124.46) (end 119.85 123.66) (width 0.2) (layer "B.Cu") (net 40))
 (segment (start 121.45 125.26) (end 120.65 124.46) (width 0.2) (layer "B.Cu") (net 40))
 (segment (start 137.63 125.26) (end 121.45 125.26) (width 0.2) (layer "B.Cu") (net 40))
 (segment (start 119.85 123.66) (end 119.85 107.48) (width 0.2) (layer "B.Cu") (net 40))
 (segment (start 138.43 124.46) (end 137.63 125.26) (width 0.2) (layer "B.Cu") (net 40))
 (segment (start 119.85 107.48) (end 120.65 106.68) (width 0.2) (layer "B.Cu") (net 40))
 (segment (start 121.45 106.348629) (end 121.45 110.96) (width 0.2) (layer "B.Cu") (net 41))
 (segment (start 120.318629 105.88) (end 120.981371 105.88) (width 0.2) (layer "B.Cu") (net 41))
 (segment (start 120.65 129.54) (end 119.45 128.34) (width 0.2) (layer "B.Cu") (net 41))
 (segment (start 156.21 128.27) (end 147.32 119.38) (width 0.2) (layer "B.Cu") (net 41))
 (segment (start 121.45 110.96) (end 120.65 111.76) (width 0.2) (layer "B.Cu") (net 41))
 (segment (start 119.45 128.34) (end 119.45 106.748629) (width 0.2) (layer "B.Cu") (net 41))
 (segment (start 120.981371 105.88) (end 121.45 106.348629) (width 0.2) (layer "B.Cu") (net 41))
 (segment (start 156.21 129.54) (end 156.21 128.27) (width 0.2) (layer "B.Cu") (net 41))
 (segment (start 138.43 128.27) (end 138.43 129.54) (width 0.2) (layer "B.Cu") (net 41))
 (segment (start 138.43 129.54) (end 137.16 129.54) (width 0.2) (layer "B.Cu") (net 41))
 (segment (start 157.01 128.74) (end 156.21 129.54) (width 0.2) (layer "B.Cu") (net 41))
 (segment (start 136.36 130.34) (end 121.45 130.34) (width 0.2) (layer "B.Cu") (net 41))
 (segment (start 156.21 123.328629) (end 157.01 124.128629) (width 0.2) (layer "B.Cu") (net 41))
 (segment (start 121.45 130.34) (end 120.65 129.54) (width 0.2) (layer "B.Cu") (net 41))
 (segment (start 156.21 111.76) (end 156.21 123.328629) (width 0.2) (layer "B.Cu") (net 41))
 (segment (start 137.16 129.54) (end 136.36 130.34) (width 0.2) (layer "B.Cu") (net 41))
 (segment (start 157.01 124.128629) (end 157.01 128.74) (width 0.2) (layer "B.Cu") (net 41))
 (segment (start 119.45 106.748629) (end 120.318629 105.88) (width 0.2) (layer "B.Cu") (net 41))
 (segment (start 147.32 119.38) (end 138.43 128.27) (width 0.2) (layer "B.Cu") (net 41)))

